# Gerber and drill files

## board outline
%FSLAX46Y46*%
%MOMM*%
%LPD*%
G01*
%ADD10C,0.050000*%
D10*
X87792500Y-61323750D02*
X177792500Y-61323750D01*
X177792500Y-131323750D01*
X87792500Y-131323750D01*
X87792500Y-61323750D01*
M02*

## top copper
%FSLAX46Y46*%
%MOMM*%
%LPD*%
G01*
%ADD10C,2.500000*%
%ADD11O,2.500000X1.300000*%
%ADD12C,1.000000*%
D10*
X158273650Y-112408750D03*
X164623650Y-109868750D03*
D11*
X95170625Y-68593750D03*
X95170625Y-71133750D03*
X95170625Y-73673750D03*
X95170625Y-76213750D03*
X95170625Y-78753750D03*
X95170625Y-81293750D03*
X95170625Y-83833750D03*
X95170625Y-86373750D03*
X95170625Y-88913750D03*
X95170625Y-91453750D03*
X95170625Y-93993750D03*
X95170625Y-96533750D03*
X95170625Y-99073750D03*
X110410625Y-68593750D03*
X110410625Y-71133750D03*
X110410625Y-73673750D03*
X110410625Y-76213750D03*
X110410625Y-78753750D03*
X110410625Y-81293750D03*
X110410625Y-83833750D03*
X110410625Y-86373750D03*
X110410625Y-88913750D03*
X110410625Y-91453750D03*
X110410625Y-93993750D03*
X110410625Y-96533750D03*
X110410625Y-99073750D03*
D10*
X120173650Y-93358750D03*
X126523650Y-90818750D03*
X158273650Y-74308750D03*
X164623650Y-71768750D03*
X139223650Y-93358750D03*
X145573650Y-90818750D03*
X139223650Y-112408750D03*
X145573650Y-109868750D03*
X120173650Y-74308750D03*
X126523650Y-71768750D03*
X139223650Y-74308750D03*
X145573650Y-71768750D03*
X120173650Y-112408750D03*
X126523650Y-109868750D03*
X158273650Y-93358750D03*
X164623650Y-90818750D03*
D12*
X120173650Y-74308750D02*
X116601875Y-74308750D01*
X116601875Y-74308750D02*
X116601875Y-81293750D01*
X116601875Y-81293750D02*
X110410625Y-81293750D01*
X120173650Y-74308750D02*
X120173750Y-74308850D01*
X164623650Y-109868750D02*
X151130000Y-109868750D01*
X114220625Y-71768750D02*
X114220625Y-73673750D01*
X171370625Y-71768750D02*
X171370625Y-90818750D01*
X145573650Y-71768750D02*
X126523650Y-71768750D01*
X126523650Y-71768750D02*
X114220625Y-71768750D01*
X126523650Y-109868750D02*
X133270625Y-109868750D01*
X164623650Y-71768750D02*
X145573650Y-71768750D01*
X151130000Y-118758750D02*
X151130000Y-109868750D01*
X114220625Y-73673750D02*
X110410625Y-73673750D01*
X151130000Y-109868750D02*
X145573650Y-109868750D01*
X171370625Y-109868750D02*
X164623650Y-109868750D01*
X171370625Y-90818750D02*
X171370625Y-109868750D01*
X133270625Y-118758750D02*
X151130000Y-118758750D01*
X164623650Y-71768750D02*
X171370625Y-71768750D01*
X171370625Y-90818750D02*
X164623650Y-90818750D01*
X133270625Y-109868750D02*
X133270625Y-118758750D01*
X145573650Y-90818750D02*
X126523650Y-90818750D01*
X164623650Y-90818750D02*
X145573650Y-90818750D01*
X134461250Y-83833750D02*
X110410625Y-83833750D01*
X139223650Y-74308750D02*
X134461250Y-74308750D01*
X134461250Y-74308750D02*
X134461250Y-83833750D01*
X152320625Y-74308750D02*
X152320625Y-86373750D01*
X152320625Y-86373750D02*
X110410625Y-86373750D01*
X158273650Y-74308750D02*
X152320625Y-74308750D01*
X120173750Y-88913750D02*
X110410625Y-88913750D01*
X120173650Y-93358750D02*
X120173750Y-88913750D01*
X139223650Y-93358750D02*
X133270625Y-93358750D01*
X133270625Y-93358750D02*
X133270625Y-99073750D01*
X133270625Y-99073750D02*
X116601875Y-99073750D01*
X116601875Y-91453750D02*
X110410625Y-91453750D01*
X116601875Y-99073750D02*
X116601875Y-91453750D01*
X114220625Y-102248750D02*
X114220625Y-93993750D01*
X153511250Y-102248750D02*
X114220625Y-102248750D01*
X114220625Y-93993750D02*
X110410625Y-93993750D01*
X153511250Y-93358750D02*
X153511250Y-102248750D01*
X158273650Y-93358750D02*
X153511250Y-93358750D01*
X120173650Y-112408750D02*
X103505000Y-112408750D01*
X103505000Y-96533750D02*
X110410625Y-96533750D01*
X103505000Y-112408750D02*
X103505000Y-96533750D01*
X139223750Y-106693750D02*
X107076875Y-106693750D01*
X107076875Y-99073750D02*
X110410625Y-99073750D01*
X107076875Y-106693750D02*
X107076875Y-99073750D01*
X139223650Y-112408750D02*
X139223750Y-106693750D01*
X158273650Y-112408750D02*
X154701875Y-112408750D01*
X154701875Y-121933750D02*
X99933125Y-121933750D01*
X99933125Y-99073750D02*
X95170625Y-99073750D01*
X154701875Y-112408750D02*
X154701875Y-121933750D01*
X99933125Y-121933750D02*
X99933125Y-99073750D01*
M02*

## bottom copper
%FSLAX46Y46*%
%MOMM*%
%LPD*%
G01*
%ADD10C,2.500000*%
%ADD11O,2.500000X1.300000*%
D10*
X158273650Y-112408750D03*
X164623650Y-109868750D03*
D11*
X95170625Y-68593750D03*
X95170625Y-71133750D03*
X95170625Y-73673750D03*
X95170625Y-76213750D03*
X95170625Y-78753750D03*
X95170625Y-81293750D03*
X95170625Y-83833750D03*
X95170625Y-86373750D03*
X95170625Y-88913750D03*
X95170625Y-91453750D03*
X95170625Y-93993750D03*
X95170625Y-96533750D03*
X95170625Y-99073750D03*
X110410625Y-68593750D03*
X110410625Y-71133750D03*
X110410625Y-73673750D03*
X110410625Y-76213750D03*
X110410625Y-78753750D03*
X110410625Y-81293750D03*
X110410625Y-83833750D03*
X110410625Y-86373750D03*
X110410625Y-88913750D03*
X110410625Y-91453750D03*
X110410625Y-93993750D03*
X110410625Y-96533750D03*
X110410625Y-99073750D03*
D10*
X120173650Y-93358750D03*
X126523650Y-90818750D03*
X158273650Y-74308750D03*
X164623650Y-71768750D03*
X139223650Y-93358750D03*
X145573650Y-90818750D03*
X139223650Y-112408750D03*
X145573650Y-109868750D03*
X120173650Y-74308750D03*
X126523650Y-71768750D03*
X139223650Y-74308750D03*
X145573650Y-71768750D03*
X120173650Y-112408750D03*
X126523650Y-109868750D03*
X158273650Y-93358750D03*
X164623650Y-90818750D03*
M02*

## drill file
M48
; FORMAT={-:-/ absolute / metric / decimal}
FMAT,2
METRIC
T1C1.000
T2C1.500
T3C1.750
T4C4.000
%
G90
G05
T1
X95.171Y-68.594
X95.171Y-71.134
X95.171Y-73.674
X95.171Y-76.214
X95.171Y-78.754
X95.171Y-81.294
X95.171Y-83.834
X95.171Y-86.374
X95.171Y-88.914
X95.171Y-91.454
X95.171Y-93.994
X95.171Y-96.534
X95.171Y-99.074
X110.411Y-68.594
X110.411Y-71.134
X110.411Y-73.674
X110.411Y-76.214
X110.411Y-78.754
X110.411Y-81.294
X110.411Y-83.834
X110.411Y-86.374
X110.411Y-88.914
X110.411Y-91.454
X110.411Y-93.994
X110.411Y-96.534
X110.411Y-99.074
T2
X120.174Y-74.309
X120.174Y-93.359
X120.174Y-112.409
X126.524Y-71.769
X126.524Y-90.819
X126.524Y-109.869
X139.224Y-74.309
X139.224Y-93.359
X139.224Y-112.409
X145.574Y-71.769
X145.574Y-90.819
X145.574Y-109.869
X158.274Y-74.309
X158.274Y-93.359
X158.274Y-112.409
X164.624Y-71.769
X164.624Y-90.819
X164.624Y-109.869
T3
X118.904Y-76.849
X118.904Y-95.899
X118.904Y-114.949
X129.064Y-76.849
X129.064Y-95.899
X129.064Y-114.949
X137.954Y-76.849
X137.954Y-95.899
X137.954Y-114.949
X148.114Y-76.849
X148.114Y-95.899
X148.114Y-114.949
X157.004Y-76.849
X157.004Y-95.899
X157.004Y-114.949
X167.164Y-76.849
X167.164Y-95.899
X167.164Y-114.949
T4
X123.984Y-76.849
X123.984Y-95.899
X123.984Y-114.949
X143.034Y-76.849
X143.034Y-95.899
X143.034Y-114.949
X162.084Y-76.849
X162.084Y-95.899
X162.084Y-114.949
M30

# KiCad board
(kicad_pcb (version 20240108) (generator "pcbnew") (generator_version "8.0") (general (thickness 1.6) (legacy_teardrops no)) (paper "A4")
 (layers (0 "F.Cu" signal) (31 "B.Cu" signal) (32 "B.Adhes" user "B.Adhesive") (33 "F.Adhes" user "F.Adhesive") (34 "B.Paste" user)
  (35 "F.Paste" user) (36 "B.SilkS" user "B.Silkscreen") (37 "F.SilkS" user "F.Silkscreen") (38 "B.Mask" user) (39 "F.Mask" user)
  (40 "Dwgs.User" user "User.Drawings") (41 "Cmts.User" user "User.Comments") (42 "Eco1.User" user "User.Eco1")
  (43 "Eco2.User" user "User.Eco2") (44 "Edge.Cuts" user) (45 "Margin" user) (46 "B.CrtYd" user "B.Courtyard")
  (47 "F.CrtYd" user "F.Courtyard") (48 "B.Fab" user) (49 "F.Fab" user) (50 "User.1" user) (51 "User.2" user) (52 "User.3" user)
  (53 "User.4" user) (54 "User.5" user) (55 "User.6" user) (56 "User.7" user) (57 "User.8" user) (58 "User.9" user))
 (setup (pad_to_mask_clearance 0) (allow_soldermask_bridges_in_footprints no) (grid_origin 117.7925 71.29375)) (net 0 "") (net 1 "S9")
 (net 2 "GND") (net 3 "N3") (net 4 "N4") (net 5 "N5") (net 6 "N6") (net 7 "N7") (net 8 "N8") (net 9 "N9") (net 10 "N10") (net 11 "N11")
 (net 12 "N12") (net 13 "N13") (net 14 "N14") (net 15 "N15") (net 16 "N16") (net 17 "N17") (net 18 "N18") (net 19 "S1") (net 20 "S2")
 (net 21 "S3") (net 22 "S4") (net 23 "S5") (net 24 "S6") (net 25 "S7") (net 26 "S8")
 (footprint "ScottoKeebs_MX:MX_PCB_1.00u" (layer "F.Cu") (at 162.08365 114.94875)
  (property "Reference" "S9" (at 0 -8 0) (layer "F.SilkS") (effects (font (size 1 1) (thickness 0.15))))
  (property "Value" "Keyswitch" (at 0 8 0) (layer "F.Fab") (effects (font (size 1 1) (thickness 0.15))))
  (pad "" np_thru_hole circle (at -5.08 0) (size 1.75 1.75) (drill 1.75) (layers "*.Cu" "*.Mask"))
  (pad "" np_thru_hole circle (at 0 0) (size 4 4) (drill 4) (layers "*.Cu" "*.Mask"))
  (pad "" np_thru_hole circle (at 5.08 0) (size 1.75 1.75) (drill 1.75) (layers "*.Cu" "*.Mask"))
  (pad "1" thru_hole circle (at -3.81 -2.54) (size 2.5 2.5) (drill 1.5) (layers "*.Cu" "*.Mask") (remove_unused_layers no) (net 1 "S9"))
  (pad "2" thru_hole circle (at 2.54 -5.08) (size 2.5 2.5) (drill 1.5) (layers "*.Cu" "*.Mask") (remove_unused_layers no) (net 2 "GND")))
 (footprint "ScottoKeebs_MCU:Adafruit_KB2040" (layer "F.Cu") (at 102.780625 83.82375)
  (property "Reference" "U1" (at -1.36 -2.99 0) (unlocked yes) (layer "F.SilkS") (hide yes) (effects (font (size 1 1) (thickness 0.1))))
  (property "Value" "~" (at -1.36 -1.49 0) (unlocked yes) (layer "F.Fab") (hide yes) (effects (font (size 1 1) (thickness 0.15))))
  (pad "1" thru_hole oval (at -7.61 -15.23 180) (size 2.5 1.3) (drill 1) (layers "*.Cu" "*.Mask") (remove_unused_layers no) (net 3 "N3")
   (solder_mask_margin 0.0508) (thermal_bridge_angle 0))
  (pad "2" thru_hole oval (at -7.61 -12.69 180) (size 2.5 1.3) (drill 1) (layers "*.Cu" "*.Mask") (remove_unused_layers no) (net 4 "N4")
   (solder_mask_margin 0.0508) (thermal_bridge_angle 0))
  (pad "3" thru_hole oval (at -7.61 -10.15 180) (size 2.5 1.3) (drill 1) (layers "*.Cu" "*.Mask") (remove_unused_layers no) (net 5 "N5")
   (solder_mask_margin 0.0508) (thermal_bridge_angle 0))
  (pad "4" thru_hole oval (at -7.61 -7.61 180) (size 2.5 1.3) (drill 1) (layers "*.Cu" "*.Mask") (remove_unused_layers no) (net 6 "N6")
   (solder_mask_margin 0.0508) (thermal_bridge_angle 0))
  (pad "5" thru_hole oval (at -7.61 -5.07 180) (size 2.5 1.3) (drill 1) (layers "*.Cu" "*.Mask") (remove_unused_layers no) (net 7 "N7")
   (solder_mask_margin 0.0508) (thermal_bridge_angle 0))
  (pad "6" thru_hole oval (at -7.61 -2.53 180) (size 2.5 1.3) (drill 1) (layers "*.Cu" "*.Mask") (remove_unused_layers no) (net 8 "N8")
   (solder_mask_margin 0.0508) (thermal_bridge_angle 0))
  (pad "7" thru_hole oval (at -7.61 0.01 180) (size 2.5 1.3) (drill 1) (layers "*.Cu" "*.Mask") (remove_unused_layers no) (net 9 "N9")
   (solder_mask_margin 0.0508) (thermal_bridge_angle 0))
  (pad "8" thru_hole oval (at -7.61 2.55 180) (size 2.5 1.3) (drill 1) (layers "*.Cu" "*.Mask") (remove_unused_layers no) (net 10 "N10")
   (solder_mask_margin 0.0508) (thermal_bridge_angle 0))
  (pad "9" thru_hole oval (at -7.61 5.09 180) (size 2.5 1.3) (drill 1) (layers "*.Cu" "*.Mask") (remove_unused_layers no) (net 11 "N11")
   (solder_mask_margin 0.0508) (thermal_bridge_angle 0))
  (pad "10" thru_hole oval (at -7.61 7.63 180) (size 2.5 1.3) (drill 1) (layers "*.Cu" "*.Mask") (remove_unused_layers no) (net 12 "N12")
   (solder_mask_margin 0.0508) (thermal_bridge_angle 0))
  (pad "11" thru_hole oval (at -7.61 10.17 180) (size 2.5 1.3) (drill 1) (layers "*.Cu" "*.Mask") (remove_unused_layers no) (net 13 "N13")
   (solder_mask_margin 0.0508) (thermal_bridge_angle 0))
  (pad "12" thru_hole oval (at -7.61 12.71 180) (size 2.5 1.3) (drill 1) (layers "*.Cu" "*.Mask") (remove_unused_layers no) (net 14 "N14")
   (solder_mask_margin 0.0508) (thermal_bridge_angle 0))
  (pad "13" thru_hole oval (at -7.61 15.25 180) (size 2.5 1.3) (drill 1) (layers "*.Cu" "*.Mask") (remove_unused_layers no) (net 1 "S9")
   (solder_mask_margin 0.0508) (thermal_bridge_angle 0))
  (pad "14" thru_hole oval (at 7.63 -15.23 180) (size 2.5 1.3) (drill 1) (layers "*.Cu" "*.Mask") (remove_unused_layers no) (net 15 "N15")
   (solder_mask_margin 0.0508) (thermal_bridge_angle 0))
  (pad "15" thru_hole oval (at 7.63 -12.69 180) (size 2.5 1.3) (drill 1) (layers "*.Cu" "*.Mask") (remove_unused_layers no) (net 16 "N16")
   (solder_mask_margin 0.0508) (thermal_bridge_angle 0))
  (pad "16" thru_hole oval (at 7.63 -10.15 180) (size 2.5 1.3) (drill 1) (layers "*.Cu" "*.Mask") (remove_unused_layers no) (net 2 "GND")
   (solder_mask_margin 0.0508) (thermal_bridge_angle 0))
  (pad "17" thru_hole oval (at 7.63 -7.61 180) (size 2.5 1.3) (drill 1) (layers "*.Cu" "*.Mask") (remove_unused_layers no) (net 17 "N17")
   (solder_mask_margin 0.0508) (thermal_bridge_angle 0))
  (pad "18" thru_hole oval (at 7.63 -5.07 180) (size 2.5 1.3) (drill 1) (layers "*.Cu" "*.Mask") (remove_unused_layers no) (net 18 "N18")
   (solder_mask_margin 0.0508) (thermal_bridge_angle 0))
  (pad "19" thru_hole oval (at 7.63 -2.53 180) (size 2.5 1.3) (drill 1) (layers "*.Cu" "*.Mask") (remove_unused_layers no) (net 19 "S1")
   (solder_mask_margin 0.0508) (thermal_bridge_angle 0))
  (pad "20" thru_hole oval (at 7.63 0.01 180) (size 2.5 1.3) (drill 1) (layers "*.Cu" "*.Mask") (remove_unused_layers no) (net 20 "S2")
   (solder_mask_margin 0.0508) (thermal_bridge_angle 0))
  (pad "21" thru_hole oval (at 7.63 2.55 180) (size 2.5 1.3) (drill 1) (layers "*.Cu" "*.Mask") (remove_unused_layers no) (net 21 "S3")
   (solder_mask_margin 0.0508) (thermal_bridge_angle 0))
  (pad "22" thru_hole oval (at 7.63 5.09 180) (size 2.5 1.3) (drill 1) (layers "*.Cu" "*.Mask") (remove_unused_layers no) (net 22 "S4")
   (solder_mask_margin 0.0508) (thermal_bridge_angle 0))
  (pad "23" thru_hole oval (at 7.63 7.63 180) (size 2.5 1.3) (drill 1) (layers "*.Cu" "*.Mask") (remove_unused_layers no) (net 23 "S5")
   (solder_mask_margin 0.0508) (thermal_bridge_angle 0))
  (pad "24" thru_hole oval (at 7.63 10.17 180) (size 2.5 1.3) (drill 1) (layers "*.Cu" "*.Mask") (remove_unused_layers no) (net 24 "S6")
   (solder_mask_margin 0.0508) (thermal_bridge_angle 0))
  (pad "25" thru_hole oval (at 7.63 12.71 180) (size 2.5 1.3) (drill 1) (layers "*.Cu" "*.Mask") (remove_unused_layers no) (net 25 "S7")
   (solder_mask_margin 0.0508) (thermal_bridge_angle 0))
  (pad "26" thru_hole oval (at 7.63 15.25 180) (size 2.5 1.3) (drill 1) (layers "*.Cu" "*.Mask") (remove_unused_layers no) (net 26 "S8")
   (solder_mask_margin 0.0508) (thermal_bridge_angle 0)))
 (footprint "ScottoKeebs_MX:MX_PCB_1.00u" (layer "F.Cu") (at 123.98365 95.89875)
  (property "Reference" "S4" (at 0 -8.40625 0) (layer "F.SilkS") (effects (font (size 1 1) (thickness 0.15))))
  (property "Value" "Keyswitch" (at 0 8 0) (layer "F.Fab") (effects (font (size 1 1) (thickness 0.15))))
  (pad "" np_thru_hole circle (at -5.08 0) (size 1.75 1.75) (drill 1.75) (layers "*.Cu" "*.Mask"))
  (pad "" np_thru_hole circle (at 0 0) (size 4 4) (drill 4) (layers "*.Cu" "*.Mask"))
  (pad "" np_thru_hole circle (at 5.08 0) (size 1.75 1.75) (drill 1.75) (layers "*.Cu" "*.Mask"))
  (pad "1" thru_hole circle (at -3.81 -2.54) (size 2.5 2.5) (drill 1.5) (layers "*.Cu" "*.Mask") (remove_unused_layers no) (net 22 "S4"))
  (pad "2" thru_hole circle (at 2.54 -5.08) (size 2.5 2.5) (drill 1.5) (layers "*.Cu" "*.Mask") (remove_unused_layers no) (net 2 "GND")))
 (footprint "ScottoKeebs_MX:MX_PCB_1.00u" (layer "F.Cu") (at 162.08365 76.84875)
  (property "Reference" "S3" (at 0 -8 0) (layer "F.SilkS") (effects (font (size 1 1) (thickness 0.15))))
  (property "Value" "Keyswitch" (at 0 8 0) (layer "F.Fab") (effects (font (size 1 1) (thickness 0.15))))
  (pad "" np_thru_hole circle (at -5.08 0) (size 1.75 1.75) (drill 1.75) (layers "*.Cu" "*.Mask"))
  (pad "" np_thru_hole circle (at 0 0) (size 4 4) (drill 4) (layers "*.Cu" "*.Mask"))
  (pad "" np_thru_hole circle (at 5.08 0) (size 1.75 1.75) (drill 1.75) (layers "*.Cu" "*.Mask"))
  (pad "1" thru_hole circle (at -3.81 -2.54) (size 2.5 2.5) (drill 1.5) (layers "*.Cu" "*.Mask") (remove_unused_layers no) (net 21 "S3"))
  (pad "2" thru_hole circle (at 2.54 -5.08) (size 2.5 2.5) (drill 1.5) (layers "*.Cu" "*.Mask") (remove_unused_layers no) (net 2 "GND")))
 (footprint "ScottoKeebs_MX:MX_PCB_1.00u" (layer "F.Cu") (at 143.03365 95.89875)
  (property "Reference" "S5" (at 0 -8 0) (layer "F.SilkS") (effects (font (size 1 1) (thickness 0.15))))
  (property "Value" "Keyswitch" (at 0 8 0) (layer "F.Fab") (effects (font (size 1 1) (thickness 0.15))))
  (pad "" np_thru_hole circle (at -5.08 0) (size 1.75 1.75) (drill 1.75) (layers "*.Cu" "*.Mask"))
  (pad "" np_thru_hole circle (at 0 0) (size 4 4) (drill 4) (layers "*.Cu" "*.Mask"))
  (pad "" np_thru_hole circle (at 5.08 0) (size 1.75 1.75) (drill 1.75) (layers "*.Cu" "*.Mask"))
  (pad "1" thru_hole circle (at -3.81 -2.54) (size 2.5 2.5) (drill 1.5) (layers "*.Cu" "*.Mask") (remove_unused_layers no) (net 23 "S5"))
  (pad "2" thru_hole circle (at 2.54 -5.08) (size 2.5 2.5) (drill 1.5) (layers "*.Cu" "*.Mask") (remove_unused_layers no) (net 2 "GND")))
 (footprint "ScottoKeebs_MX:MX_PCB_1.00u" (layer "F.Cu") (at 143.03365 114.94875)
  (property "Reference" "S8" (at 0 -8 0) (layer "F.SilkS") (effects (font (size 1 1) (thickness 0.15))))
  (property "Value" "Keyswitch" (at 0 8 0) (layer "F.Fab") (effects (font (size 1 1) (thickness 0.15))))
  (pad "" np_thru_hole circle (at -5.08 0) (size 1.75 1.75) (drill 1.75) (layers "*.Cu" "*.Mask"))
  (pad "" np_thru_hole circle (at 0 0) (size 4 4) (drill 4) (layers "*.Cu" "*.Mask"))
  (pad "" np_thru_hole circle (at 5.08 0) (size 1.75 1.75) (drill 1.75) (layers "*.Cu" "*.Mask"))
  (pad "1" thru_hole circle (at -3.81 -2.54) (size 2.5 2.5) (drill 1.5) (layers "*.Cu" "*.Mask") (remove_unused_layers no) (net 26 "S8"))
  (pad "2" thru_hole circle (at 2.54 -5.08) (size 2.5 2.5) (drill 1.5) (layers "*.Cu" "*.Mask") (remove_unused_layers no) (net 2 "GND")))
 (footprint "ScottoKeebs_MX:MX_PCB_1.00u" (layer "F.Cu") (at 123.98365 76.84875)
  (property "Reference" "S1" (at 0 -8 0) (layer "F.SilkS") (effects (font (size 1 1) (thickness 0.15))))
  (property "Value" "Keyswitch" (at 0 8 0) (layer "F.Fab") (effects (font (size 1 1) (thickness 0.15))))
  (pad "" np_thru_hole circle (at -5.08 0) (size 1.75 1.75) (drill 1.75) (layers "*.Cu" "*.Mask"))
  (pad "" np_thru_hole circle (at 0 0) (size 4 4) (drill 4) (layers "*.Cu" "*.Mask"))
  (pad "" np_thru_hole circle (at 5.08 0) (size 1.75 1.75) (drill 1.75) (layers "*.Cu" "*.Mask"))
  (pad "1" thru_hole circle (at -3.81 -2.54) (size 2.5 2.5) (drill 1.5) (layers "*.Cu" "*.Mask") (remove_unused_layers no) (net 19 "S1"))
  (pad "2" thru_hole circle (at 2.54 -5.08) (size 2.5 2.5) (drill 1.5) (layers "*.Cu" "*.Mask") (remove_unused_layers no) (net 2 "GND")))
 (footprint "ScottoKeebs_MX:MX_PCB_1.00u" (layer "F.Cu") (at 143.03365 76.84875)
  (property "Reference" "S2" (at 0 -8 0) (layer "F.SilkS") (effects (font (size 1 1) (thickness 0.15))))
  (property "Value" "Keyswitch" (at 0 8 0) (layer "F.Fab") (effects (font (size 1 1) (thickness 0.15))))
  (pad "" np_thru_hole circle (at -5.08 0) (size 1.75 1.75) (drill 1.75) (layers "*.Cu" "*.Mask"))
  (pad "" np_thru_hole circle (at 0 0) (size 4 4) (drill 4) (layers "*.Cu" "*.Mask"))
  (pad "" np_thru_hole circle (at 5.08 0) (size 1.75 1.75) (drill 1.75) (layers "*.Cu" "*.Mask"))
  (pad "1" thru_hole circle (at -3.81 -2.54) (size 2.5 2.5) (drill 1.5) (layers "*.Cu" "*.Mask") (remove_unused_layers no) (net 20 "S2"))
  (pad "2" thru_hole circle (at 2.54 -5.08) (size 2.5 2.5) (drill 1.5) (layers "*.Cu" "*.Mask") (remove_unused_layers no) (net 2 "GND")))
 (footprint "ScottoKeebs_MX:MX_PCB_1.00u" (layer "F.Cu") (at 123.98365 114.94875)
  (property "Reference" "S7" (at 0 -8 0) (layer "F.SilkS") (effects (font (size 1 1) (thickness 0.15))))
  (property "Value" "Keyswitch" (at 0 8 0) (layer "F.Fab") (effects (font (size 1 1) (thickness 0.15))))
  (pad "" np_thru_hole circle (at -5.08 0) (size 1.75 1.75) (drill 1.75) (layers "*.Cu" "*.Mask"))
  (pad "" np_thru_hole circle (at 0 0) (size 4 4) (drill 4) (layers "*.Cu" "*.Mask"))
  (pad "" np_thru_hole circle (at 5.08 0) (size 1.75 1.75) (drill 1.75) (layers "*.Cu" "*.Mask"))
  (pad "1" thru_hole circle (at -3.81 -2.54) (size 2.5 2.5) (drill 1.5) (layers "*.Cu" "*.Mask") (remove_unused_layers no) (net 25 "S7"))
  (pad "2" thru_hole circle (at 2.54 -5.08) (size 2.5 2.5) (drill 1.5) (layers "*.Cu" "*.Mask") (remove_unused_layers no) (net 2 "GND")))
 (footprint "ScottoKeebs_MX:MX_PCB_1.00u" (layer "F.Cu") (at 162.08365 95.89875)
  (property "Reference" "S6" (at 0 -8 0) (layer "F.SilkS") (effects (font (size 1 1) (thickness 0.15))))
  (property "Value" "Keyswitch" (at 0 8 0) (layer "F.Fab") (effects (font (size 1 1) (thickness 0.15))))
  (pad "" np_thru_hole circle (at -5.08 0) (size 1.75 1.75) (drill 1.75) (layers "*.Cu" "*.Mask"))
  (pad "" np_thru_hole circle (at 0 0) (size 4 4) (drill 4) (layers "*.Cu" "*.Mask"))
  (pad "" np_thru_hole circle (at 5.08 0) (size 1.75 1.75) (drill 1.75) (layers "*.Cu" "*.Mask"))
  (pad "1" thru_hole circle (at -3.81 -2.54) (size 2.5 2.5) (drill 1.5) (layers "*.Cu" "*.Mask") (remove_unused_layers no) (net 24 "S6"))
  (pad "2" thru_hole circle (at 2.54 -5.08) (size 2.5 2.5) (drill 1.5) (layers "*.Cu" "*.Mask") (remove_unused_layers no) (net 2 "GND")))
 (gr_rect (start 87.7925 61.32375) (end 177.7925 131.32375) (stroke (width 0.05) (type default)) (fill none) (layer "Edge.Cuts"))
 (segment (start 120.17365 74.30875) (end 116.601875 74.30875) (width 1) (layer "F.Cu") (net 19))
 (segment (start 116.601875 74.30875) (end 116.601875 81.29375) (width 1) (layer "F.Cu") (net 19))
 (segment (start 116.601875 81.29375) (end 110.410625 81.29375) (width 1) (layer "F.Cu") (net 19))
 (segment (start 120.17365 74.30875) (end 120.17375 74.30885) (width 1) (layer "F.Cu") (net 19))
 (segment (start 164.62365 109.86875) (end 151.13 109.86875) (width 1) (layer "F.Cu") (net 2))
 (segment (start 114.220625 71.76875) (end 114.220625 73.67375) (width 1) (layer "F.Cu") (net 2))
 (segment (start 171.370625 71.76875) (end 171.370625 90.81875) (width 1) (layer "F.Cu") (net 2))
 (segment (start 145.57365 71.76875) (end 126.52365 71.76875) (width 1) (layer "F.Cu") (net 2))
 (segment (start 126.52365 71.76875) (end 114.220625 71.76875) (width 1) (layer "F.Cu") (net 2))
 (segment (start 126.52365 109.86875) (end 133.270625 109.86875) (width 1) (layer "F.Cu") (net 2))
 (segment (start 164.62365 71.76875) (end 145.57365 71.76875) (width 1) (layer "F.Cu") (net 2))
 (segment (start 151.13 118.75875) (end 151.13 109.86875) (width 1) (layer "F.Cu") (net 2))
 (segment (start 114.220625 73.67375) (end 110.410625 73.67375) (width 1) (layer "F.Cu") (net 2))
 (segment (start 151.13 109.86875) (end 145.57365 109.86875) (width 1) (layer "F.Cu") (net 2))
 (segment (start 171.370625 109.86875) (end 164.62365 109.86875) (width 1) (layer "F.Cu") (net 2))
 (segment (start 171.370625 90.81875) (end 171.370625 109.86875) (width 1) (layer "F.Cu") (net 2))
 (segment (start 133.270625 118.75875) (end 151.13 118.75875) (width 1) (layer "F.Cu") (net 2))
 (segment (start 164.62365 71.76875) (end 171.370625 71.76875) (width 1) (layer "F.Cu") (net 2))
 (segment (start 171.370625 90.81875) (end 164.62365 90.81875) (width 1) (layer "F.Cu") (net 2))
 (segment (start 133.270625 109.86875) (end 133.270625 118.75875) (width 1) (layer "F.Cu") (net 2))
 (segment (start 145.57365 90.81875) (end 126.52365 90.81875) (width 1) (layer "F.Cu") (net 2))
 (segment (start 164.62365 90.81875) (end 145.57365 90.81875) (width 1) (layer "F.Cu") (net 2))
 (segment (start 134.46125 83.83375) (end 110.410625 83.83375) (width 1) (layer "F.Cu") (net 20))
 (segment (start 139.22365 74.30875) (end 134.46125 74.30875) (width 1) (layer "F.Cu") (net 20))
 (segment (start 134.46125 74.30875) (end 134.46125 83.83375) (width 1) (layer "F.Cu") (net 20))
 (segment (start 152.320625 74.30875) (end 152.320625 86.37375) (width 1) (layer "F.Cu") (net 21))
 (segment (start 152.320625 86.37375) (end 110.410625 86.37375) (width 1) (layer "F.Cu") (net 21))
 (segment (start 158.27365 74.30875) (end 152.320625 74.30875) (width 1) (layer "F.Cu") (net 21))
 (segment (start 120.17375 88.91375) (end 110.410625 88.91375) (width 1) (layer "F.Cu") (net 22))
 (segment (start 120.17365 93.35875) (end 120.17375 88.91375) (width 1) (layer "F.Cu") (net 22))
 (segment (start 139.22365 93.35875) (end 133.270625 93.35875) (width 1) (layer "F.Cu") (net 23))
 (segment (start 133.270625 93.35875) (end 133.270625 99.07375) (width 1) (layer "F.Cu") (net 23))
 (segment (start 133.270625 99.07375) (end 116.601875 99.07375) (width 1) (layer "F.Cu") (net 23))
 (segment (start 116.601875 91.45375) (end 110.410625 91.45375) (width 1) (layer "F.Cu") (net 23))
 (segment (start 116.601875 99.07375) (end 116.601875 91.45375) (width 1) (layer "F.Cu") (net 23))
 (segment (start 114.220625 102.24875) (end 114.220625 93.99375) (width 1) (layer "F.Cu") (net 24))
 (segment (start 153.51125 102.24875) (end 114.220625 102.24875) (width 1) (layer "F.Cu") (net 24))
 (segment (start 114.220625 93.99375) (end 110.410625 93.99375) (width 1) (layer "F.Cu") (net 24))
 (segment (start 153.51125 93.35875) (end 153.51125 102.24875) (width 1) (layer "F.Cu") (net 24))
 (segment (start 158.27365 93.35875) (end 153.51125 93.35875) (width 1) (layer "F.Cu") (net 24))
 (segment (start 120.17365 112.40875) (end 103.505 112.40875) (width 1) (layer "F.Cu") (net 25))
 (segment (start 103.505 96.53375) (end 110.410625 96.53375) (width 1) (layer "F.Cu") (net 25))
 (segment (start 103.505 112.40875) (end 103.505 96.53375) (width 1) (layer "F.Cu") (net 25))
 (segment (start 139.22375 106.69375) (end 107.076875 106.69375) (width 1) (layer "F.Cu") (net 26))
 (segment (start 107.076875 99.07375) (end 110.410625 99.07375) (width 1) (layer "F.Cu") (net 26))
 (segment (start 107.076875 106.69375) (end 107.076875 99.07375) (width 1) (layer "F.Cu") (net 26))
 (segment (start 139.22365 112.40875) (end 139.22375 106.69375) (width 1) (layer "F.Cu") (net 26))
 (segment (start 158.27365 112.40875) (end 154.701875 112.40875) (width 1) (layer "F.Cu") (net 1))
 (segment (start 154.701875 121.93375) (end 99.933125 121.93375) (width 1) (layer "F.Cu") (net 1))
 (segment (start 99.933125 99.07375) (end 95.170625 99.07375) (width 1) (layer "F.Cu") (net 1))
 (segment (start 154.701875 112.40875) (end 154.701875 121.93375) (width 1) (layer "F.Cu") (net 1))
 (segment (start 99.933125 121.93375) (end 99.933125 99.07375) (width 1) (layer "F.Cu") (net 1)))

